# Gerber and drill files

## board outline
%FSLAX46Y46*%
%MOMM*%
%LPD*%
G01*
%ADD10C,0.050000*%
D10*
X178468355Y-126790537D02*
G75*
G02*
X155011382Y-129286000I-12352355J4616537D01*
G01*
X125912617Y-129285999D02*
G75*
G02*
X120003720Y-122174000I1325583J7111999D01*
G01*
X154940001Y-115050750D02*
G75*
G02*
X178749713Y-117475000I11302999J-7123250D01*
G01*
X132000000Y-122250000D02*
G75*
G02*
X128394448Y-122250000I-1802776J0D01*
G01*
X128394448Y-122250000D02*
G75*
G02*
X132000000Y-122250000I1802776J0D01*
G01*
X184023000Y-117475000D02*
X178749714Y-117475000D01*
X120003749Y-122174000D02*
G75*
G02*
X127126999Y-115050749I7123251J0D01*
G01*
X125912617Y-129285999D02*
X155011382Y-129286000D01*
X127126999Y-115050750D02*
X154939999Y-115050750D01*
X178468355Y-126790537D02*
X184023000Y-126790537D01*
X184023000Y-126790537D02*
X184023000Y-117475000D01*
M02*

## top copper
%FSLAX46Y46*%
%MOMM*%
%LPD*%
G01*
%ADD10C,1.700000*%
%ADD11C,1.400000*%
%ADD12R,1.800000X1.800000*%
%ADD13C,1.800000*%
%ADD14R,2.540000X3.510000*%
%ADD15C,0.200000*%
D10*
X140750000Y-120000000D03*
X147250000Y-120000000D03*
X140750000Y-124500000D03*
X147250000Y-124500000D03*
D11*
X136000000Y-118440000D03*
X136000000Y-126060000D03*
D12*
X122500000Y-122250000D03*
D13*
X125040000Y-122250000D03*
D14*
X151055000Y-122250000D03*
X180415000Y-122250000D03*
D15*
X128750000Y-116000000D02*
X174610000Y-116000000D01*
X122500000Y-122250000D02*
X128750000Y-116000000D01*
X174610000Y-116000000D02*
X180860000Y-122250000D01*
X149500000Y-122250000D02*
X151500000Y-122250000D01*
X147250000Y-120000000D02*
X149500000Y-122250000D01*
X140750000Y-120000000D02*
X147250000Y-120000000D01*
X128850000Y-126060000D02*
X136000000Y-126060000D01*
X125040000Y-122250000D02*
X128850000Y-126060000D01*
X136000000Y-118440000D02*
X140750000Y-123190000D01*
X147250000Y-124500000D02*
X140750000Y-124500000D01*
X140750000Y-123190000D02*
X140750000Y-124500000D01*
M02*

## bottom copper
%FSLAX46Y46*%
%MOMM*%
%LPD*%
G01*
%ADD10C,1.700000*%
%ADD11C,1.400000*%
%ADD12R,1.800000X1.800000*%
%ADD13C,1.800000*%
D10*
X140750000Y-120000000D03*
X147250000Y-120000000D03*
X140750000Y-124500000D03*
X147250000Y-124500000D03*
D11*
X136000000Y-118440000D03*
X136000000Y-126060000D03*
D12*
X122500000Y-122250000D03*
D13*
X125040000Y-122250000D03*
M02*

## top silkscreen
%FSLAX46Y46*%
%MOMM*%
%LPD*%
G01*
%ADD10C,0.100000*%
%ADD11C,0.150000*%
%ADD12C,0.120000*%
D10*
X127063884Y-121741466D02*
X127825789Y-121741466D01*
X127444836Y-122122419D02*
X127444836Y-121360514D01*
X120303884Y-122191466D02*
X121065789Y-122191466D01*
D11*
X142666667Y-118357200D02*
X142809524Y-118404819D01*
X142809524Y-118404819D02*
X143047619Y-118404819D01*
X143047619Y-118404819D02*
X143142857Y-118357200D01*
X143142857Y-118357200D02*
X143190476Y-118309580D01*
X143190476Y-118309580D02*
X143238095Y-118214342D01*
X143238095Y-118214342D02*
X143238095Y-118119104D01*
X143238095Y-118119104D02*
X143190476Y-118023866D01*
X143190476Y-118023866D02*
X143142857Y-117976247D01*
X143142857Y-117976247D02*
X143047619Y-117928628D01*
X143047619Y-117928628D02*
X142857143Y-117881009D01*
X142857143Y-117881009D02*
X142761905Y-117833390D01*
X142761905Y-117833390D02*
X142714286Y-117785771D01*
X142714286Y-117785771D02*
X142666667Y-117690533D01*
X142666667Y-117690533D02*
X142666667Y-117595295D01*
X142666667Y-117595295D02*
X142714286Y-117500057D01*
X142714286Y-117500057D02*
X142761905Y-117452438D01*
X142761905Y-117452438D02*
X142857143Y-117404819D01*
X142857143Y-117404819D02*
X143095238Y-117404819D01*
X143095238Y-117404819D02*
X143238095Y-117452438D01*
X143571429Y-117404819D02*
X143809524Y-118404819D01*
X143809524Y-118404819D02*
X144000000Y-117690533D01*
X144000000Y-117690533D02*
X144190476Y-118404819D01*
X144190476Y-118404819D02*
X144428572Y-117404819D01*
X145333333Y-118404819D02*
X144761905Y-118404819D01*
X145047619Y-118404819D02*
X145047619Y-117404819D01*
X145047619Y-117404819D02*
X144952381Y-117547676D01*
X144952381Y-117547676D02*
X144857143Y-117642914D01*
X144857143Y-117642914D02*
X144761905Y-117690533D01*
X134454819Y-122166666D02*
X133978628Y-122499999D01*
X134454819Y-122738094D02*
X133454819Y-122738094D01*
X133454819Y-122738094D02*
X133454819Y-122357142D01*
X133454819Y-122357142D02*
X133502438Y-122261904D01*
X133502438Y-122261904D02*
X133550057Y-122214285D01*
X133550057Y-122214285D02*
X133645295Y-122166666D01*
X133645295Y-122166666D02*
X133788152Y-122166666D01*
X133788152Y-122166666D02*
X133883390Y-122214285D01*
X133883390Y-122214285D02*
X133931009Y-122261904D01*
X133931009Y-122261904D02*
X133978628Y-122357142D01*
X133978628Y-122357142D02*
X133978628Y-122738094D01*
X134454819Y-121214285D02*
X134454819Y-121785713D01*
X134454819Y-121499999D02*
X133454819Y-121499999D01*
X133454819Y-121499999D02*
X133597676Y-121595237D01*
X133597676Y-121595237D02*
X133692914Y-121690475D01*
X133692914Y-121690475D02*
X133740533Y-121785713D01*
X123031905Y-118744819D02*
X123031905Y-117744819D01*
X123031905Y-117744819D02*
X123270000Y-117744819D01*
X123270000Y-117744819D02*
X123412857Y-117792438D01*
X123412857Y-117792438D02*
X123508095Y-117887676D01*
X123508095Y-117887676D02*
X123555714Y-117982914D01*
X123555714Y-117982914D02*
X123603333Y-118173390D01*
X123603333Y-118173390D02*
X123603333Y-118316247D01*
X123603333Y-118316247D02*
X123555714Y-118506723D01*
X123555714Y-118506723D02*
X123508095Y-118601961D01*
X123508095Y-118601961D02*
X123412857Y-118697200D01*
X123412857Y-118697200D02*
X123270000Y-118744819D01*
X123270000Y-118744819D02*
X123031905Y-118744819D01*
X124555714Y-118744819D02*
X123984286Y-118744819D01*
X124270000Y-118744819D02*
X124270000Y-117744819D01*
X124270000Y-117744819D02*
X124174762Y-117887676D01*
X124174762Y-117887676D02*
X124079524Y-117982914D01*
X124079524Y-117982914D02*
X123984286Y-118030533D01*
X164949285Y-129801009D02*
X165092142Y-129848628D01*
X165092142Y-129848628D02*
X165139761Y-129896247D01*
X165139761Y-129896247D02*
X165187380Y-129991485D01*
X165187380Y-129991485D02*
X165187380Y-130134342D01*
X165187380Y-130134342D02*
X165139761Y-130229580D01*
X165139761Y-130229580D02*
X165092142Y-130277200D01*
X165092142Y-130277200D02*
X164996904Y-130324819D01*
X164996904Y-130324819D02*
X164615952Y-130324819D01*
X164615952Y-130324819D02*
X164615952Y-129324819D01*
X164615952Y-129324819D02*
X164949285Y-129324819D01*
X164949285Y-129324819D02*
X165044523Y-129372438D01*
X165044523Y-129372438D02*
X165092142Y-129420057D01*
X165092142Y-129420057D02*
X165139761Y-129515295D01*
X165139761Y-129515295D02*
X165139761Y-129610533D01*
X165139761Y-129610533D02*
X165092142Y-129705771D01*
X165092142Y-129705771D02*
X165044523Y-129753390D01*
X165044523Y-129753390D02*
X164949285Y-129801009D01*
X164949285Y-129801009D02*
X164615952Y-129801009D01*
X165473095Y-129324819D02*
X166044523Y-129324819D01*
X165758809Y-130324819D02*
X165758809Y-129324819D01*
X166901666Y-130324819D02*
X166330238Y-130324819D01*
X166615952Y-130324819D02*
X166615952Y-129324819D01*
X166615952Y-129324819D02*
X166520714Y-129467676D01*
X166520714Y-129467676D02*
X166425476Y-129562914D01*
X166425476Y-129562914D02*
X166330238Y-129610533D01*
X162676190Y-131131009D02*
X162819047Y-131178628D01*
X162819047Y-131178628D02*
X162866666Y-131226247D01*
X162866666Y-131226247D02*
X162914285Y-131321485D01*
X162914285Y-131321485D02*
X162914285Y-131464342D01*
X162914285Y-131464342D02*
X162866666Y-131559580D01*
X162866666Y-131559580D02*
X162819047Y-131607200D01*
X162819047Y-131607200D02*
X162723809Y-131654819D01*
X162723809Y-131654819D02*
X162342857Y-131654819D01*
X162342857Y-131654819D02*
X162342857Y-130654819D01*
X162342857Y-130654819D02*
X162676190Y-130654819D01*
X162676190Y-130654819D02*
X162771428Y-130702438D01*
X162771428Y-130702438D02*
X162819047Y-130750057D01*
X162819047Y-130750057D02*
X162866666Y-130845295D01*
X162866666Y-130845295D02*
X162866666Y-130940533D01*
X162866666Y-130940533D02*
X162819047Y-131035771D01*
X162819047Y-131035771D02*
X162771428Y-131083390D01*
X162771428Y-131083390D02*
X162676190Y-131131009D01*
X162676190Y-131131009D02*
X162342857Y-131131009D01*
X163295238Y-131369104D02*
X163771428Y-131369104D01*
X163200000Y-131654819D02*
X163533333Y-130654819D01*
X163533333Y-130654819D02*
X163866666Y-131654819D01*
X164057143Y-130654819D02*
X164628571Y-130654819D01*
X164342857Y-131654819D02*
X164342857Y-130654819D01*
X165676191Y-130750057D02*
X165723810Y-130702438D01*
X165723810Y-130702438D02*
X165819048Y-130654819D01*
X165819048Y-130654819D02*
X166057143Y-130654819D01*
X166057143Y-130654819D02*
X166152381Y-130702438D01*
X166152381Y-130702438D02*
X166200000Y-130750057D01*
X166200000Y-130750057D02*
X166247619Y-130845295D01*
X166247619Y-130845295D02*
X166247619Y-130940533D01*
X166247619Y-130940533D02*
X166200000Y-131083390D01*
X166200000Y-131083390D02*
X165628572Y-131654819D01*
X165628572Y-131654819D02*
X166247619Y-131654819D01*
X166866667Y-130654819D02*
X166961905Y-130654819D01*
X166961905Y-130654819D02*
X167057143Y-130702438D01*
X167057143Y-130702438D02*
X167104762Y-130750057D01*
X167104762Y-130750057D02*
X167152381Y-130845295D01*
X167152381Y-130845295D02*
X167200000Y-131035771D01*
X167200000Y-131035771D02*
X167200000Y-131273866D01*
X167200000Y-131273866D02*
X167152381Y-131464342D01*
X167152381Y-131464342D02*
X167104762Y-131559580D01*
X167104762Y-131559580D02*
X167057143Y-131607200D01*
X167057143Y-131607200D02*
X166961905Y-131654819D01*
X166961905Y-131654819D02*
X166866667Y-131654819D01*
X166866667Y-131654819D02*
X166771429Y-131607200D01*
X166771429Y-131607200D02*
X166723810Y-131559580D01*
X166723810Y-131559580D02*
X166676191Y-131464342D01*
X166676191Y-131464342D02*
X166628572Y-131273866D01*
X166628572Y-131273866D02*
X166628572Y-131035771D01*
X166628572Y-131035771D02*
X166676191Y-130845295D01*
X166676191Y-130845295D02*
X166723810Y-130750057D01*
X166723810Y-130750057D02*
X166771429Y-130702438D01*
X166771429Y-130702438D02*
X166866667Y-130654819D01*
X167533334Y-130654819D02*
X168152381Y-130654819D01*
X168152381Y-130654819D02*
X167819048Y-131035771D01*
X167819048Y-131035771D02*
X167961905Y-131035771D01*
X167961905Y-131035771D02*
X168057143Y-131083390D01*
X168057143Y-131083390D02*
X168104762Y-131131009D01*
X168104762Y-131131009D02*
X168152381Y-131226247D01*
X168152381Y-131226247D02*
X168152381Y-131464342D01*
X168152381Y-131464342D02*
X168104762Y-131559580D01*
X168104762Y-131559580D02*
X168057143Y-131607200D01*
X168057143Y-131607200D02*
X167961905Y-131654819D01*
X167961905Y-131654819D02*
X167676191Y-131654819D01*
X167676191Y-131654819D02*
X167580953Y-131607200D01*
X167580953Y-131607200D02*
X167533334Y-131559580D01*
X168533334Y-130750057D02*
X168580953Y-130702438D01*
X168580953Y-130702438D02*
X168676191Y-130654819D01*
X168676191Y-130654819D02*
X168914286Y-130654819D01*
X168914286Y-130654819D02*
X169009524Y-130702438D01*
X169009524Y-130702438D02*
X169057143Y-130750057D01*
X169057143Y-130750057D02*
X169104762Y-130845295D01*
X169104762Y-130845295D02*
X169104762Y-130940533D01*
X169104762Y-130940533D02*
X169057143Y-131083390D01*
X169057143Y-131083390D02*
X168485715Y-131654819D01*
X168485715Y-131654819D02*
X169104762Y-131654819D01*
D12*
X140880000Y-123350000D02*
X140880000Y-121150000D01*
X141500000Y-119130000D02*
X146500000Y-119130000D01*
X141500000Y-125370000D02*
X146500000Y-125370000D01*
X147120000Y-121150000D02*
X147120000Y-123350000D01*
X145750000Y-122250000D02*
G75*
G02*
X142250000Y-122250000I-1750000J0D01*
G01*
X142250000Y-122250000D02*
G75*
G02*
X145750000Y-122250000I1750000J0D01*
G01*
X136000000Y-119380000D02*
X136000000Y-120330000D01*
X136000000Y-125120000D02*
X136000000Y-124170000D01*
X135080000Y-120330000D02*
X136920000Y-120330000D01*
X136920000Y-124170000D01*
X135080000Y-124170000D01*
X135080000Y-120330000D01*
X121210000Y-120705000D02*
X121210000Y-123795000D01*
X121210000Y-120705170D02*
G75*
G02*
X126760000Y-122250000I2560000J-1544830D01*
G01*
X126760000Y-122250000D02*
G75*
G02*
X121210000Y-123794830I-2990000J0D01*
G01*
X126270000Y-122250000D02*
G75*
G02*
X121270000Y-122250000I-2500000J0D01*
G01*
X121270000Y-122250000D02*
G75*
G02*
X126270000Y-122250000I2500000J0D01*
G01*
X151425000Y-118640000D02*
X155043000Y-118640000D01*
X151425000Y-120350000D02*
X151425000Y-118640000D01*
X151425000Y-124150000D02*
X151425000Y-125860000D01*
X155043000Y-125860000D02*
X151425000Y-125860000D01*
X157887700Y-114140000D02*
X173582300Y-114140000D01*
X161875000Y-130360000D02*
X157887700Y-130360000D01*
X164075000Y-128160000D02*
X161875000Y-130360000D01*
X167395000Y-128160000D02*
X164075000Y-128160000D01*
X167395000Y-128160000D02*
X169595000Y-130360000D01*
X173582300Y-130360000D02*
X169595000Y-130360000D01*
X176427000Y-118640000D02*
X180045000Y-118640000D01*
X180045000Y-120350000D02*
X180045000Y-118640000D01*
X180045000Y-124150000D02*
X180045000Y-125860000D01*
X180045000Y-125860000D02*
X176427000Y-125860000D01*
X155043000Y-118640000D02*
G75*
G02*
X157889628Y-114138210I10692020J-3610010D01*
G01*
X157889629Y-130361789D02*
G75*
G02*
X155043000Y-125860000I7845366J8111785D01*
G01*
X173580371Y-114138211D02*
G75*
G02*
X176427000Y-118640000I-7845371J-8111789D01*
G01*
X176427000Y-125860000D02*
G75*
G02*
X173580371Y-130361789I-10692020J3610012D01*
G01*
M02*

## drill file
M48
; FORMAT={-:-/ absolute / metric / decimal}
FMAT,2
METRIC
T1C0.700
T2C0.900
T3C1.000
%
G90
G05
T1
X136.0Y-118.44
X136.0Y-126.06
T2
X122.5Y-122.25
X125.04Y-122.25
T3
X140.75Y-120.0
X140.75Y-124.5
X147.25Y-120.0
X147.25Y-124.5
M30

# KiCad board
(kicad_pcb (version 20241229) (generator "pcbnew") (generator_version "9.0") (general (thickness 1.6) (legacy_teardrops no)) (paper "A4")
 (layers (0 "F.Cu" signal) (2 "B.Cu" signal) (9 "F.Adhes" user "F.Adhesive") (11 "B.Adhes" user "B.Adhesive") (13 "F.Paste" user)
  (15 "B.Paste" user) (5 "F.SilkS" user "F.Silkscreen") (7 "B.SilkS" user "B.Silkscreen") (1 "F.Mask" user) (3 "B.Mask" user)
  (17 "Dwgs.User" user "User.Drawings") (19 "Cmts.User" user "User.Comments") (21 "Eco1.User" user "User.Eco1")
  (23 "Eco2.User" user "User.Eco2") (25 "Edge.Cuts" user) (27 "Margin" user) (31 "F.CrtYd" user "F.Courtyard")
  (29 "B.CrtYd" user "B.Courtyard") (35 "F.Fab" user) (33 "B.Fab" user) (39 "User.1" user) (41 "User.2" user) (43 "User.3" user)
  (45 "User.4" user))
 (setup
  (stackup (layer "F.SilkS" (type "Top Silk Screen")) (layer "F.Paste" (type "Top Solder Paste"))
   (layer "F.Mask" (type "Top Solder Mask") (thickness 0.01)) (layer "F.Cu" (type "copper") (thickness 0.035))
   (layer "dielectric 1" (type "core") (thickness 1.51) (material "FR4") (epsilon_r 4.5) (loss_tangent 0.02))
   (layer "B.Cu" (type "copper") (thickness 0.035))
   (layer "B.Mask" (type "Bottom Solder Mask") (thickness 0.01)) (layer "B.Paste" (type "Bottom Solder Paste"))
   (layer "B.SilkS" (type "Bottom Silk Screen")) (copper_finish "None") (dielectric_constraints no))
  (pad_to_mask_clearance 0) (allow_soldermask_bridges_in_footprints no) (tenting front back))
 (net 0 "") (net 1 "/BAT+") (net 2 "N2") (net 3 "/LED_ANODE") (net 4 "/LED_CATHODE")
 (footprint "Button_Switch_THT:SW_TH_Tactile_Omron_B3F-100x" (layer "F.Cu") (at 140.75 120)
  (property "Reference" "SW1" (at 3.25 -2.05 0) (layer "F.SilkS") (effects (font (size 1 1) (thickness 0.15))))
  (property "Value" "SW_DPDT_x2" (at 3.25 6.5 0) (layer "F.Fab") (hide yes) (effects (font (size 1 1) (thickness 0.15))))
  (fp_line (start 0.13 3.35) (end 0.13 1.15) (stroke (width 0.12) (type solid)) (layer "F.SilkS"))
  (fp_line (start 0.75 -0.87) (end 5.75 -0.87) (stroke (width 0.12) (type solid)) (layer "F.SilkS"))
  (fp_line (start 0.75 5.37) (end 5.75 5.37) (stroke (width 0.12) (type solid)) (layer "F.SilkS"))
  (fp_line (start 6.37 1.15) (end 6.37 3.35) (stroke (width 0.12) (type solid)) (layer "F.SilkS"))
  (fp_circle (center 3.25 2.25) (end 5 2.25) (stroke (width 0.12) (type solid)) (fill no) (layer "F.SilkS"))
  (pad "1" thru_hole circle (at 0 0) (size 1.7 1.7) (drill 1) (layers "*.Cu" "*.Mask") (remove_unused_layers no) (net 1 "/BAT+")
   (thermal_bridge_angle 90))
  (pad "1" thru_hole circle (at 6.5 0) (size 1.7 1.7) (drill 1) (layers "*.Cu" "*.Mask") (remove_unused_layers no) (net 1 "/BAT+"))
  (pad "2" thru_hole circle (at 0 4.5) (size 1.7 1.7) (drill 1) (layers "*.Cu" "*.Mask") (remove_unused_layers no) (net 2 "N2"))
  (pad "2" thru_hole circle (at 6.5 4.5) (size 1.7 1.7) (drill 1) (layers "*.Cu" "*.Mask") (remove_unused_layers no) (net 2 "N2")))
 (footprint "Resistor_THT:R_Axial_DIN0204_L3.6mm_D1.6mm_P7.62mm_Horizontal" (layer "F.Cu") (at 136 118.44 -90)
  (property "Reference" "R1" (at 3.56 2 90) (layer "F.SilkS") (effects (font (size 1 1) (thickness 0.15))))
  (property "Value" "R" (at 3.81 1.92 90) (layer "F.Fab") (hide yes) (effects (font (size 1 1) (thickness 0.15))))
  (fp_line (start 0.94 0) (end 1.89 0) (stroke (width 0.12) (type solid)) (layer "F.SilkS"))
  (fp_line (start 6.68 0) (end 5.73 0) (stroke (width 0.12) (type solid)) (layer "F.SilkS"))
  (fp_rect (start 1.89 -0.92) (end 5.73 0.92) (stroke (width 0.12) (type solid)) (fill no) (layer "F.SilkS"))
  (pad "1" thru_hole circle (at 0 0 270) (size 1.4 1.4) (drill 0.7) (layers "*.Cu" "*.Mask") (remove_unused_layers no) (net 2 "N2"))
  (pad "2" thru_hole circle (at 7.62 0 270) (size 1.4 1.4) (drill 0.7) (layers "*.Cu" "*.Mask") (remove_unused_layers no)
   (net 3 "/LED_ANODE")))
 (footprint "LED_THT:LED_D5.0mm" (layer "F.Cu") (at 122.5 122.25)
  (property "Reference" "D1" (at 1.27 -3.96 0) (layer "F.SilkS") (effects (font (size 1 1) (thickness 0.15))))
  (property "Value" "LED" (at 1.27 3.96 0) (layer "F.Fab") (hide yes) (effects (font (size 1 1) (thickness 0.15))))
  (fp_line (start -1.29 -1.545) (end -1.29 1.545) (stroke (width 0.12) (type solid)) (layer "F.SilkS"))
  (fp_arc (start -1.29 -1.54483) (mid 2.071779 -2.880495) (end 4.26 0) (stroke (width 0.12) (type solid)) (layer "F.SilkS"))
  (fp_arc (start 4.26 0) (mid 2.071779 2.880495) (end -1.29 1.54483) (stroke (width 0.12) (type solid)) (layer "F.SilkS"))
  (fp_circle (center 1.27 0) (end 3.77 0) (stroke (width 0.12) (type solid)) (fill no) (layer "F.SilkS"))
  (pad "1" thru_hole rect (at 0 0) (size 1.8 1.8) (drill 0.9) (layers "*.Cu" "*.Mask") (remove_unused_layers no) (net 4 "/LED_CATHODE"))
  (pad "2" thru_hole circle (at 2.54 0) (size 1.8 1.8) (drill 0.9) (layers "*.Cu" "*.Mask") (remove_unused_layers no) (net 3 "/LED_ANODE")))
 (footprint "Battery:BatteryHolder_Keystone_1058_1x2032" (layer "F.Cu") (at 165.735 122.25)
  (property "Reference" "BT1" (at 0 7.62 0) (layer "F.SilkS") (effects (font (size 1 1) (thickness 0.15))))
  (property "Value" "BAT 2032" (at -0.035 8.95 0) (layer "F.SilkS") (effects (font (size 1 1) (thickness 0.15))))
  (fp_line (start -14.31 -3.61) (end -10.692 -3.61) (stroke (width 0.12) (type solid)) (layer "F.SilkS"))
  (fp_line (start -14.31 -1.9) (end -14.31 -3.61) (stroke (width 0.12) (type solid)) (layer "F.SilkS"))
  (fp_line (start -14.31 1.9) (end -14.31 3.61) (stroke (width 0.12) (type solid)) (layer "F.SilkS"))
  (fp_line (start -10.692 3.61) (end -14.31 3.61) (stroke (width 0.12) (type solid)) (layer "F.SilkS"))
  (fp_line (start -7.8473 -8.11) (end 7.8473 -8.11) (stroke (width 0.12) (type solid)) (layer "F.SilkS"))
  (fp_line (start -3.86 8.11) (end -7.8473 8.11) (stroke (width 0.12) (type solid)) (layer "F.SilkS"))
  (fp_line (start -1.66 5.91) (end -3.86 8.11) (stroke (width 0.12) (type solid)) (layer "F.SilkS"))
  (fp_line (start 1.66 5.91) (end -1.66 5.91) (stroke (width 0.12) (type solid)) (layer "F.SilkS"))
  (fp_line (start 1.66 5.91) (end 3.86 8.11) (stroke (width 0.12) (type solid)) (layer "F.SilkS"))
  (fp_line (start 7.8473 8.11) (end 3.86 8.11) (stroke (width 0.12) (type solid)) (layer "F.SilkS"))
  (fp_line (start 10.692 -3.61) (end 14.31 -3.61) (stroke (width 0.12) (type solid)) (layer "F.SilkS"))
  (fp_line (start 14.31 -1.9) (end 14.31 -3.61) (stroke (width 0.12) (type solid)) (layer "F.SilkS"))
  (fp_line (start 14.31 1.9) (end 14.31 3.61) (stroke (width 0.12) (type solid)) (layer "F.SilkS"))
  (fp_line (start 14.31 3.61) (end 10.692 3.61) (stroke (width 0.12) (type solid)) (layer "F.SilkS"))
  (fp_arc (start -10.692 -3.61) (mid -9.538084 -6.031244) (end -7.845371 -8.111789) (stroke (width 0.12) (type solid)) (layer "F.SilkS"))
  (fp_arc (start -7.845371 8.111789) (mid -9.538085 6.031244) (end -10.692 3.61) (stroke (width 0.12) (type solid)) (layer "F.SilkS"))
  (fp_arc (start 7.845371 -8.111789) (mid 9.538085 -6.031244) (end 10.692 -3.61) (stroke (width 0.12) (type solid)) (layer "F.SilkS"))
  (fp_arc (start 10.692 3.61) (mid 9.538084 6.031244) (end 7.845371 8.111789) (stroke (width 0.12) (type solid)) (layer "F.SilkS"))
  (pad "1" smd rect (at -14.68 0) (size 2.54 3.51) (layers "F.Cu" "F.Mask" "F.Paste") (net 1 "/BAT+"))
  (pad "2" smd rect (at 14.68 0) (size 2.54 3.51) (layers "F.Cu" "F.Mask" "F.Paste") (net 4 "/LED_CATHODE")))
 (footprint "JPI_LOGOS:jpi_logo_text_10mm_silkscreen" (layer "B.Cu") (at 165.8 127 180)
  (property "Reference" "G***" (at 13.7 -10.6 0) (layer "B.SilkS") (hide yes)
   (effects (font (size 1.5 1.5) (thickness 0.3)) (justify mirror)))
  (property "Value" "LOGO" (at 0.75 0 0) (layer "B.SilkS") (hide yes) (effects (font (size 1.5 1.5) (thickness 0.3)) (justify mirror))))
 (gr_arc (start 178.468355 126.790537) (mid 167.511007 135.286858) (end 155.011382 129.286) (stroke (width 0.05) (type default))
  (layer "Edge.Cuts"))
 (gr_arc (start 125.912617 129.285999) (mid 121.673706 126.797182) (end 120.003749 122.174) (stroke (width 0.05) (type default))
  (layer "Edge.Cuts"))
 (gr_arc (start 154.940001 115.05075) (mid 167.596321 108.882386) (end 178.749713 117.475) (stroke (width 0.05) (type default))
  (layer "Edge.Cuts"))
 (gr_circle (center 130.197224 122.25) (end 131.197224 123.75) (stroke (width 0.05) (type default)) (fill no) (layer "Edge.Cuts"))
 (gr_line (start 184.023 117.475) (end 178.749714 117.475) (stroke (width 0.05) (type default)) (layer "Edge.Cuts"))
 (gr_arc (start 120.003749 122.174) (mid 122.090101 117.137102) (end 127.126999 115.05075) (stroke (width 0.05) (type default))
  (layer "Edge.Cuts"))
 (gr_line (start 125.912617 129.285999) (end 155.011382 129.286) (stroke (width 0.05) (type default)) (layer "Edge.Cuts"))
 (gr_line (start 127.126999 115.05075) (end 154.939999 115.05075) (stroke (width 0.05) (type default)) (layer "Edge.Cuts"))
 (gr_line (start 178.468355 126.790537) (end 184.023 126.790537) (stroke (width 0.05) (type default)) (layer "Edge.Cuts"))
 (gr_line (start 184.023 126.790537) (end 184.023 117.475) (stroke (width 0.05) (type default)) (layer "Edge.Cuts"))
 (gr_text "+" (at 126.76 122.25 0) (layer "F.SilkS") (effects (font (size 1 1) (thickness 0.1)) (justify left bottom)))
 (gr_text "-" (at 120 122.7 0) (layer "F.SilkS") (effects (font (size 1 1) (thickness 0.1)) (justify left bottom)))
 (segment (start 128.75 116) (end 174.61 116) (width 0.2) (layer "F.Cu") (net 4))
 (segment (start 122.5 122.25) (end 128.75 116) (width 0.2) (layer "F.Cu") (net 4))
 (segment (start 174.61 116) (end 180.86 122.25) (width 0.2) (layer "F.Cu") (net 4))
 (segment (start 149.5 122.25) (end 151.5 122.25) (width 0.2) (layer "F.Cu") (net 1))
 (segment (start 147.25 120) (end 149.5 122.25) (width 0.2) (layer "F.Cu") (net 1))
 (segment (start 140.75 120) (end 147.25 120) (width 0.2) (layer "F.Cu") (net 1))
 (segment (start 128.85 126.06) (end 136 126.06) (width 0.2) (layer "F.Cu") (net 3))
 (segment (start 125.04 122.25) (end 128.85 126.06) (width 0.2) (layer "F.Cu") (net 3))
 (segment (start 136 118.44) (end 140.75 123.19) (width 0.2) (layer "F.Cu") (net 2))
 (segment (start 147.25 124.5) (end 140.75 124.5) (width 0.2) (layer "F.Cu") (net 2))
 (segment (start 140.75 123.19) (end 140.75 124.5) (width 0.2) (layer "F.Cu") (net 2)))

